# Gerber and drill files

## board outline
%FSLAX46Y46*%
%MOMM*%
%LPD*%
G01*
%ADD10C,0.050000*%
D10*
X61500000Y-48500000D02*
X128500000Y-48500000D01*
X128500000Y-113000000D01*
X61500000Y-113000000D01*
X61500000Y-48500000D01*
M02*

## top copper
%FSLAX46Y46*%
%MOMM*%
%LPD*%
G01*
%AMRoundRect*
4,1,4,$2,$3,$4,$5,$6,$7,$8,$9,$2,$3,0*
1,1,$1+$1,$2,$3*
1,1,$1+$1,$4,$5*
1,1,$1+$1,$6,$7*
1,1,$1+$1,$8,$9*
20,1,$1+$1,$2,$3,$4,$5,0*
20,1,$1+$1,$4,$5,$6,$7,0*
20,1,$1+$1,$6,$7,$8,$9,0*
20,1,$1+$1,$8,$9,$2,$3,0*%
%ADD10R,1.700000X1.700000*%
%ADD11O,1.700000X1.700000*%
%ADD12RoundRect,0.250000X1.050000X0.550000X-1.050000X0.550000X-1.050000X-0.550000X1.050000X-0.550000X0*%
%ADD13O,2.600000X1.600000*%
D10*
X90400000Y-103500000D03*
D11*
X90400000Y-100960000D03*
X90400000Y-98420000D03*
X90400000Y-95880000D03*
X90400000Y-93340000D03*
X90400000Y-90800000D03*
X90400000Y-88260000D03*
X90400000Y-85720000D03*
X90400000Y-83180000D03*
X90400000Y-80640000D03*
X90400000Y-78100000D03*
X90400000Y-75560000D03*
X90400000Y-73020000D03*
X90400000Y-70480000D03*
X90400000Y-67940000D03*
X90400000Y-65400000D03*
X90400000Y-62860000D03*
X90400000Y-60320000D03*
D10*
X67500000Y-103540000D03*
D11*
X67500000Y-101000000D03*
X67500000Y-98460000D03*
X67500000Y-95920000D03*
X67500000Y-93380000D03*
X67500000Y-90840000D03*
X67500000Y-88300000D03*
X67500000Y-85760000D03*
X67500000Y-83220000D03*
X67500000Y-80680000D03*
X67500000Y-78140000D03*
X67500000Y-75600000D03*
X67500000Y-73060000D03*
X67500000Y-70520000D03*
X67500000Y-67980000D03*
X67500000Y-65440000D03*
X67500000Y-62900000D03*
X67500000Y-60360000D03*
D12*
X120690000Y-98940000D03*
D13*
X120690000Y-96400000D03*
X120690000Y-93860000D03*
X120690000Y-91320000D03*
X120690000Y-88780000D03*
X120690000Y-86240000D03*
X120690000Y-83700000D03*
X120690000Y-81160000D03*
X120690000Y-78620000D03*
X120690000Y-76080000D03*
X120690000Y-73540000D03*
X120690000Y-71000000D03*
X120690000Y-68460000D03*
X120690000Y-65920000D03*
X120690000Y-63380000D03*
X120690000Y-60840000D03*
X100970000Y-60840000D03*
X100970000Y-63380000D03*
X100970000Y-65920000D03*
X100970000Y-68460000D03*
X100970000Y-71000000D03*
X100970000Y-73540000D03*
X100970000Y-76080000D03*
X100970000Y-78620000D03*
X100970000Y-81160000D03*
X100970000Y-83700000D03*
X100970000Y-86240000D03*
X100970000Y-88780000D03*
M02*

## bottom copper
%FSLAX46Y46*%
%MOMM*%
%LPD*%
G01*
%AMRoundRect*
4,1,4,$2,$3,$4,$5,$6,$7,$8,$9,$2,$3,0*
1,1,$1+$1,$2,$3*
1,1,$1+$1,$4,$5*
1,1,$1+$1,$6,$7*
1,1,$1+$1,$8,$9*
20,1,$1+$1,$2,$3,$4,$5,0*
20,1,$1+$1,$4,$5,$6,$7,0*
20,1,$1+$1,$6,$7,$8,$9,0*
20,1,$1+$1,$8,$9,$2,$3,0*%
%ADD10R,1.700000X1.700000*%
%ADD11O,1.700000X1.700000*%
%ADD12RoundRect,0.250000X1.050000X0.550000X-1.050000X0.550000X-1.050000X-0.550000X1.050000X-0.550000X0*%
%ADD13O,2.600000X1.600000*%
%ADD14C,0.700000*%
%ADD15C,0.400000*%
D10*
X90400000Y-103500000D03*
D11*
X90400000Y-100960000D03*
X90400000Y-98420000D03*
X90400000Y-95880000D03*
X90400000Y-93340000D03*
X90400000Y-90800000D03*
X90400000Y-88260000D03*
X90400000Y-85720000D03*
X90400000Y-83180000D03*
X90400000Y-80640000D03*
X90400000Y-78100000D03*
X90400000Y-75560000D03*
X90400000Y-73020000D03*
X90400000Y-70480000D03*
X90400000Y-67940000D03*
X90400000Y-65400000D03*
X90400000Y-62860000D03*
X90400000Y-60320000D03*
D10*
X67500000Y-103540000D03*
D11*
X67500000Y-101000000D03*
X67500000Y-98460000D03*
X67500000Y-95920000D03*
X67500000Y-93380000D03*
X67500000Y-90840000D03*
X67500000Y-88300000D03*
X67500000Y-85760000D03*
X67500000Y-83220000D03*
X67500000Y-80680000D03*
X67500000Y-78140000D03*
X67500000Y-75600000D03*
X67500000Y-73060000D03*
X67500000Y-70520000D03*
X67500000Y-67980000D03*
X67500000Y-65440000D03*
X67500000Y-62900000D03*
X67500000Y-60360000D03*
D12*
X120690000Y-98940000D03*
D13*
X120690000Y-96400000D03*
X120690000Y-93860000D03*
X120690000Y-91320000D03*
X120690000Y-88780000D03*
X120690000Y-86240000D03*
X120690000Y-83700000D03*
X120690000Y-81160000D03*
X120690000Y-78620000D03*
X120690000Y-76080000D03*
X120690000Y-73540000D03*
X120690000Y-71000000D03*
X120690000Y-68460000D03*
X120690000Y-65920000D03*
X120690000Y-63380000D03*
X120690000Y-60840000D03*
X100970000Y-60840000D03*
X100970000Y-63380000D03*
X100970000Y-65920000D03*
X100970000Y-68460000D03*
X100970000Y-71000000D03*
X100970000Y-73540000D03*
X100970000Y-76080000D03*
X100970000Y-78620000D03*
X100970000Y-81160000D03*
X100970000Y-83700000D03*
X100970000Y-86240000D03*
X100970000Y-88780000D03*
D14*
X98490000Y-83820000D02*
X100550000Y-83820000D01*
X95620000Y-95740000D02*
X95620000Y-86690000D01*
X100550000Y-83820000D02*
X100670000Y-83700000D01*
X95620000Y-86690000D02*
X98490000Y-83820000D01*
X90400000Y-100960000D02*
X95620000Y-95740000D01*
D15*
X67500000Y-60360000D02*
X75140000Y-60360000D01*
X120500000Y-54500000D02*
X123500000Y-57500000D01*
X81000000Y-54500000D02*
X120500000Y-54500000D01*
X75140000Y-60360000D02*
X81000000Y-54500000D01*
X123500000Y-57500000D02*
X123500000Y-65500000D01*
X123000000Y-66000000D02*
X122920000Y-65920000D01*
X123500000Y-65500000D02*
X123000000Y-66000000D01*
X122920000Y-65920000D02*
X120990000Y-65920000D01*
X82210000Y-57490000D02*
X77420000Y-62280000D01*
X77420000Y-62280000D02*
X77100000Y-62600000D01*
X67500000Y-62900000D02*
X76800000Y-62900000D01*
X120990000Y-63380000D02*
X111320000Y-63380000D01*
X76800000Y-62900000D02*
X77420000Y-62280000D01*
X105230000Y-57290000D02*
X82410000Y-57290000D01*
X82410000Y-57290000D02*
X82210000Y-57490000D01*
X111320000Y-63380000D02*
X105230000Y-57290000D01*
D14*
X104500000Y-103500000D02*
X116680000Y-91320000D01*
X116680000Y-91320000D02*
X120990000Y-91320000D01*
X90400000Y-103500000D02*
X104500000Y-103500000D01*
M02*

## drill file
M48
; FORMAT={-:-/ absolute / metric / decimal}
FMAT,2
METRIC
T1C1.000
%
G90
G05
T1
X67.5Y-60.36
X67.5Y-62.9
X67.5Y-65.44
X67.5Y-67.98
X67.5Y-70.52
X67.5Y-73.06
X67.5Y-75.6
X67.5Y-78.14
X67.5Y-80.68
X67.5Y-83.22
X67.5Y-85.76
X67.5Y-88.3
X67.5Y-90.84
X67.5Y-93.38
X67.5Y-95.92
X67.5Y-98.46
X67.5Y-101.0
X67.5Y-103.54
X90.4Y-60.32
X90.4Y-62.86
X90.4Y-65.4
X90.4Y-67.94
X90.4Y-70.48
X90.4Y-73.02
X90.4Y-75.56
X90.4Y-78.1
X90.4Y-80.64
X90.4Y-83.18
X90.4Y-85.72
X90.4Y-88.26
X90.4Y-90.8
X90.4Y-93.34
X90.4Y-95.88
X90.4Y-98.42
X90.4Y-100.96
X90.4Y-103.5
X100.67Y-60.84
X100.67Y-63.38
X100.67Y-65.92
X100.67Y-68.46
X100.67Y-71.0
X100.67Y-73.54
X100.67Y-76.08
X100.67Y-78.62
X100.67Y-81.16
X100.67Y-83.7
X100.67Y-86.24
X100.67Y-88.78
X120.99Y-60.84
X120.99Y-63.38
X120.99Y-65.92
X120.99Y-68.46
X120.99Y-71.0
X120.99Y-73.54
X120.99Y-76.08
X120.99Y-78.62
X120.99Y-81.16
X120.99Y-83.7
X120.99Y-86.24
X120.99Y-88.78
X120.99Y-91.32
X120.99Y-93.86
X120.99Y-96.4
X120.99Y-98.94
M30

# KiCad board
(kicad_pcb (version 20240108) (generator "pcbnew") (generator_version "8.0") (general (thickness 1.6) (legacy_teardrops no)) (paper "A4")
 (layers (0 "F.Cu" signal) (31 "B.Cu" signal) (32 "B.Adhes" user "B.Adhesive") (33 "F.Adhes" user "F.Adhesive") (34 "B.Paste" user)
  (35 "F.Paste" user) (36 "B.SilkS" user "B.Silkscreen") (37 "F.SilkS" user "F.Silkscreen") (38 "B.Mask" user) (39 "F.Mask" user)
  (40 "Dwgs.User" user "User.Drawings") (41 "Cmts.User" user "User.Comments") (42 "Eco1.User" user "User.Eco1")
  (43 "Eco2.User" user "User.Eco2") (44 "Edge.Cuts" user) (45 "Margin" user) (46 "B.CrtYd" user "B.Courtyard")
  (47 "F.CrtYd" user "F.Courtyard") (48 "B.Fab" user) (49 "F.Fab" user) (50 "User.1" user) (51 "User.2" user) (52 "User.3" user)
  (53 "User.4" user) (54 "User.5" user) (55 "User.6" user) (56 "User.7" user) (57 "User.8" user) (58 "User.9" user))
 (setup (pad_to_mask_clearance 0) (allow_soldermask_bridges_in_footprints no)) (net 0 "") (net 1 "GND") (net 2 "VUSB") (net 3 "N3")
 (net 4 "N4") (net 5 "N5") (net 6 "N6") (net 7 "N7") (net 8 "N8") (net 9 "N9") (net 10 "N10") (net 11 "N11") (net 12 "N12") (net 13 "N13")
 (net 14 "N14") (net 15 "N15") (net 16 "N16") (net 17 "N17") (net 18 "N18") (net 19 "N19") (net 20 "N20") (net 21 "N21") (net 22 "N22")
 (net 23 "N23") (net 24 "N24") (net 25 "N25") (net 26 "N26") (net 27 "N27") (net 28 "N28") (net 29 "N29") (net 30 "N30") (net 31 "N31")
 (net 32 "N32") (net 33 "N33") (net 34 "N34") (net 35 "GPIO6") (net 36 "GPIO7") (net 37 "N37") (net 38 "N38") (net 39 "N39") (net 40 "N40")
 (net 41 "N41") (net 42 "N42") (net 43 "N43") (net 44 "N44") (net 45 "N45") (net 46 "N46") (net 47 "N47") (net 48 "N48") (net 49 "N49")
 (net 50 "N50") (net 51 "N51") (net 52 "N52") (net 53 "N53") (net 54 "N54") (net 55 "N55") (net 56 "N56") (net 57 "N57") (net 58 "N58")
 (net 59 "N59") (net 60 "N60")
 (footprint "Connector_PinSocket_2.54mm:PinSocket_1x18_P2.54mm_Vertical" (layer "F.Cu") (at 90.4 103.5 180)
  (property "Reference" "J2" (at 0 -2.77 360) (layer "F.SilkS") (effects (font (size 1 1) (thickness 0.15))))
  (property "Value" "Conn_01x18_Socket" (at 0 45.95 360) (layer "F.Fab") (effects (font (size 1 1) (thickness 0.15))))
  (pad "1" thru_hole rect (at 0 0 180) (size 1.7 1.7) (drill 1) (layers "*.Cu" "*.Mask") (remove_unused_layers no) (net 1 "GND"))
  (pad "2" thru_hole oval (at 0 2.54 180) (size 1.7 1.7) (drill 1) (layers "*.Cu" "*.Mask") (remove_unused_layers no) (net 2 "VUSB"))
  (pad "3" thru_hole oval (at 0 5.08 180) (size 1.7 1.7) (drill 1) (layers "*.Cu" "*.Mask") (remove_unused_layers no) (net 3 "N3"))
  (pad "4" thru_hole oval (at 0 7.62 180) (size 1.7 1.7) (drill 1) (layers "*.Cu" "*.Mask") (remove_unused_layers no) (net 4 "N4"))
  (pad "5" thru_hole oval (at 0 10.16 180) (size 1.7 1.7) (drill 1) (layers "*.Cu" "*.Mask") (remove_unused_layers no) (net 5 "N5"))
  (pad "6" thru_hole oval (at 0 12.7 180) (size 1.7 1.7) (drill 1) (layers "*.Cu" "*.Mask") (remove_unused_layers no) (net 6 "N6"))
  (pad "7" thru_hole oval (at 0 15.24 180) (size 1.7 1.7) (drill 1) (layers "*.Cu" "*.Mask") (remove_unused_layers no) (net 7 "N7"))
  (pad "8" thru_hole oval (at 0 17.78 180) (size 1.7 1.7) (drill 1) (layers "*.Cu" "*.Mask") (remove_unused_layers no) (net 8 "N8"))
  (pad "9" thru_hole oval (at 0 20.32 180) (size 1.7 1.7) (drill 1) (layers "*.Cu" "*.Mask") (remove_unused_layers no) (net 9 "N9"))
  (pad "10" thru_hole oval (at 0 22.86 180) (size 1.7 1.7) (drill 1) (layers "*.Cu" "*.Mask") (remove_unused_layers no) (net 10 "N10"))
  (pad "11" thru_hole oval (at 0 25.4 180) (size 1.7 1.7) (drill 1) (layers "*.Cu" "*.Mask") (remove_unused_layers no) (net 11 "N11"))
  (pad "12" thru_hole oval (at 0 27.94 180) (size 1.7 1.7) (drill 1) (layers "*.Cu" "*.Mask") (remove_unused_layers no) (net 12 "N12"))
  (pad "13" thru_hole oval (at 0 30.48 180) (size 1.7 1.7) (drill 1) (layers "*.Cu" "*.Mask") (remove_unused_layers no) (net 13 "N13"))
  (pad "14" thru_hole oval (at 0 33.02 180) (size 1.7 1.7) (drill 1) (layers "*.Cu" "*.Mask") (remove_unused_layers no) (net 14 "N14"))
  (pad "15" thru_hole oval (at 0 35.56 180) (size 1.7 1.7) (drill 1) (layers "*.Cu" "*.Mask") (remove_unused_layers no) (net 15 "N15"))
  (pad "16" thru_hole oval (at 0 38.1 180) (size 1.7 1.7) (drill 1) (layers "*.Cu" "*.Mask") (remove_unused_layers no) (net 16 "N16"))
  (pad "17" thru_hole oval (at 0 40.64 180) (size 1.7 1.7) (drill 1) (layers "*.Cu" "*.Mask") (remove_unused_layers no) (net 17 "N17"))
  (pad "18" thru_hole oval (at 0 43.18 180) (size 1.7 1.7) (drill 1) (layers "*.Cu" "*.Mask") (remove_unused_layers no) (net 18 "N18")))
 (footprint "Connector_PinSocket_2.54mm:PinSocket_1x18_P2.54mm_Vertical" (layer "F.Cu") (at 67.5 103.54 180)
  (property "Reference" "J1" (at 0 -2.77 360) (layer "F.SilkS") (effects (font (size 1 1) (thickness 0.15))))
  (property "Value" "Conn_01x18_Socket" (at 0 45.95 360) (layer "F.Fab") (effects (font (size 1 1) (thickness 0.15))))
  (pad "1" thru_hole rect (at 0 0 180) (size 1.7 1.7) (drill 1) (layers "*.Cu" "*.Mask") (remove_unused_layers no) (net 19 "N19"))
  (pad "2" thru_hole oval (at 0 2.54 180) (size 1.7 1.7) (drill 1) (layers "*.Cu" "*.Mask") (remove_unused_layers no) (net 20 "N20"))
  (pad "3" thru_hole oval (at 0 5.08 180) (size 1.7 1.7) (drill 1) (layers "*.Cu" "*.Mask") (remove_unused_layers no) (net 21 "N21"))
  (pad "4" thru_hole oval (at 0 7.62 180) (size 1.7 1.7) (drill 1) (layers "*.Cu" "*.Mask") (remove_unused_layers no) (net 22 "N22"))
  (pad "5" thru_hole oval (at 0 10.16 180) (size 1.7 1.7) (drill 1) (layers "*.Cu" "*.Mask") (remove_unused_layers no) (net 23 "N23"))
  (pad "6" thru_hole oval (at 0 12.7 180) (size 1.7 1.7) (drill 1) (layers "*.Cu" "*.Mask") (remove_unused_layers no) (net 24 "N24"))
  (pad "7" thru_hole oval (at 0 15.24 180) (size 1.7 1.7) (drill 1) (layers "*.Cu" "*.Mask") (remove_unused_layers no) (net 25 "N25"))
  (pad "8" thru_hole oval (at 0 17.78 180) (size 1.7 1.7) (drill 1) (layers "*.Cu" "*.Mask") (remove_unused_layers no) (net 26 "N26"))
  (pad "9" thru_hole oval (at 0 20.32 180) (size 1.7 1.7) (drill 1) (layers "*.Cu" "*.Mask") (remove_unused_layers no) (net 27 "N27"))
  (pad "10" thru_hole oval (at 0 22.86 180) (size 1.7 1.7) (drill 1) (layers "*.Cu" "*.Mask") (remove_unused_layers no) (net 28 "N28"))
  (pad "11" thru_hole oval (at 0 25.4 180) (size 1.7 1.7) (drill 1) (layers "*.Cu" "*.Mask") (remove_unused_layers no) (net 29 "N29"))
  (pad "12" thru_hole oval (at 0 27.94 180) (size 1.7 1.7) (drill 1) (layers "*.Cu" "*.Mask") (remove_unused_layers no) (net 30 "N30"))
  (pad "13" thru_hole oval (at 0 30.48 180) (size 1.7 1.7) (drill 1) (layers "*.Cu" "*.Mask") (remove_unused_layers no) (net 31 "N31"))
  (pad "14" thru_hole oval (at 0 33.02 180) (size 1.7 1.7) (drill 1) (layers "*.Cu" "*.Mask") (remove_unused_layers no) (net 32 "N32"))
  (pad "15" thru_hole oval (at 0 35.56 180) (size 1.7 1.7) (drill 1) (layers "*.Cu" "*.Mask") (remove_unused_layers no) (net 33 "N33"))
  (pad "16" thru_hole oval (at 0 38.1 180) (size 1.7 1.7) (drill 1) (layers "*.Cu" "*.Mask") (remove_unused_layers no) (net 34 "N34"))
  (pad "17" thru_hole oval (at 0 40.64 180) (size 1.7 1.7) (drill 1) (layers "*.Cu" "*.Mask") (remove_unused_layers no) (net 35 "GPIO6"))
  (pad "18" thru_hole oval (at 0 43.18 180) (size 1.7 1.7) (drill 1) (layers "*.Cu" "*.Mask") (remove_unused_layers no) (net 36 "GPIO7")))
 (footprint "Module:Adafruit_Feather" (layer "F.Cu") (at 120.99 98.94 180)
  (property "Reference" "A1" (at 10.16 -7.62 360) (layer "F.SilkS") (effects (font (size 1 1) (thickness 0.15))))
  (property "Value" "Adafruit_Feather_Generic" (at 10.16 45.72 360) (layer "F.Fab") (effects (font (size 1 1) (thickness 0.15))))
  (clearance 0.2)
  (pad "1" thru_hole roundrect (at 0 0 180) (size 2.6 1.6) (drill 1 (offset 0.3 0)) (layers "*.Cu" "*.Mask") (remove_unused_layers no)
   (roundrect_rratio 0.15625) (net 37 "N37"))
  (pad "2" thru_hole oval (at 0 2.54 180) (size 2.6 1.6) (drill 1 (offset 0.3 0)) (layers "*.Cu" "*.Mask") (remove_unused_layers no)
   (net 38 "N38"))
  (pad "3" thru_hole oval (at 0 5.08 180) (size 2.6 1.6) (drill 1 (offset 0.3 0)) (layers "*.Cu" "*.Mask") (remove_unused_layers no)
   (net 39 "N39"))
  (pad "4" thru_hole oval (at 0 7.62 180) (size 2.6 1.6) (drill 1 (offset 0.3 0)) (layers "*.Cu" "*.Mask") (remove_unused_layers no)
   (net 1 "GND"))
  (pad "5" thru_hole oval (at 0 10.16 180) (size 2.6 1.6) (drill 1 (offset 0.3 0)) (layers "*.Cu" "*.Mask") (remove_unused_layers no)
   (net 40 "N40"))
  (pad "6" thru_hole oval (at 0 12.7 180) (size 2.6 1.6) (drill 1 (offset 0.3 0)) (layers "*.Cu" "*.Mask") (remove_unused_layers no)
   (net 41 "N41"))
  (pad "7" thru_hole oval (at 0 15.24 180) (size 2.6 1.6) (drill 1 (offset 0.3 0)) (layers "*.Cu" "*.Mask") (remove_unused_layers no)
   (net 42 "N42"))
  (pad "8" thru_hole oval (at 0 17.78 180) (size 2.6 1.6) (drill 1 (offset 0.3 0)) (layers "*.Cu" "*.Mask") (remove_unused_layers no)
   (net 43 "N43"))
  (pad "9" thru_hole oval (at 0 20.32 180) (size 2.6 1.6) (drill 1 (offset 0.3 0)) (layers "*.Cu" "*.Mask") (remove_unused_layers no)
   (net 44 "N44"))
  (pad "10" thru_hole oval (at 0 22.86 180) (size 2.6 1.6) (drill 1 (offset 0.3 0)) (layers "*.Cu" "*.Mask") (remove_unused_layers no)
   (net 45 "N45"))
  (pad "11" thru_hole oval (at 0 25.4 180) (size 2.6 1.6) (drill 1 (offset 0.3 0)) (layers "*.Cu" "*.Mask") (remove_unused_layers no)
   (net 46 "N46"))
  (pad "12" thru_hole oval (at 0 27.94 180) (size 2.6 1.6) (drill 1 (offset 0.3 0)) (layers "*.Cu" "*.Mask") (remove_unused_layers no)
   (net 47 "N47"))
  (pad "13" thru_hole oval (at 0 30.48 180) (size 2.6 1.6) (drill 1 (offset 0.3 0)) (layers "*.Cu" "*.Mask") (remove_unused_layers no)
   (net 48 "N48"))
  (pad "14" thru_hole oval (at 0 33.02 180) (size 2.6 1.6) (drill 1 (offset 0.3 0)) (layers "*.Cu" "*.Mask") (remove_unused_layers no)
   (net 36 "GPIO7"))
  (pad "15" thru_hole oval (at 0 35.56 180) (size 2.6 1.6) (drill 1 (offset 0.3 0)) (layers "*.Cu" "*.Mask") (remove_unused_layers no)
   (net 35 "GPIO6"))
  (pad "16" thru_hole oval (at 0 38.1 180) (size 2.6 1.6) (drill 1 (offset 0.3 0)) (layers "*.Cu" "*.Mask") (remove_unused_layers no)
   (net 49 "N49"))
  (pad "17" thru_hole oval (at 20.32 38.1) (size 2.6 1.6) (drill 1 (offset 0.3 0)) (layers "*.Cu" "*.Mask") (remove_unused_layers no)
   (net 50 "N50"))
  (pad "18" thru_hole oval (at 20.32 35.56) (size 2.6 1.6) (drill 1 (offset 0.3 0)) (layers "*.Cu" "*.Mask") (remove_unused_layers no)
   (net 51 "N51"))
  (pad "19" thru_hole oval (at 20.32 33.02) (size 2.6 1.6) (drill 1 (offset 0.3 0)) (layers "*.Cu" "*.Mask") (remove_unused_layers no)
   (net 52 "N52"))
  (pad "20" thru_hole oval (at 20.32 30.48) (size 2.6 1.6) (drill 1 (offset 0.3 0)) (layers "*.Cu" "*.Mask") (remove_unused_layers no)
   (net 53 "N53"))
  (pad "21" thru_hole oval (at 20.32 27.94) (size 2.6 1.6) (drill 1 (offset 0.3 0)) (layers "*.Cu" "*.Mask") (remove_unused_layers no)
   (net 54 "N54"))
  (pad "22" thru_hole oval (at 20.32 25.4) (size 2.6 1.6) (drill 1 (offset 0.3 0)) (layers "*.Cu" "*.Mask") (remove_unused_layers no)
   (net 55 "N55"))
  (pad "23" thru_hole oval (at 20.32 22.86) (size 2.6 1.6) (drill 1 (offset 0.3 0)) (layers "*.Cu" "*.Mask") (remove_unused_layers no)
   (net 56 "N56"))
  (pad "24" thru_hole oval (at 20.32 20.32) (size 2.6 1.6) (drill 1 (offset 0.3 0)) (layers "*.Cu" "*.Mask") (remove_unused_layers no)
   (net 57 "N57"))
  (pad "25" thru_hole oval (at 20.32 17.78) (size 2.6 1.6) (drill 1 (offset 0.3 0)) (layers "*.Cu" "*.Mask") (remove_unused_layers no)
   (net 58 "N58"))
  (pad "26" thru_hole oval (at 20.32 15.24) (size 2.6 1.6) (drill 1 (offset 0.3 0)) (layers "*.Cu" "*.Mask") (remove_unused_layers no)
   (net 2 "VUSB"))
  (pad "27" thru_hole oval (at 20.32 12.7) (size 2.6 1.6) (drill 1 (offset 0.3 0)) (layers "*.Cu" "*.Mask") (remove_unused_layers no)
   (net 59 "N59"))
  (pad "28" thru_hole oval (at 20.32 10.16) (size 2.6 1.6) (drill 1 (offset 0.3 0)) (layers "*.Cu" "*.Mask") (remove_unused_layers no)
   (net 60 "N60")))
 (gr_rect (start 61.5 48.5) (end 128.5 113) (stroke (width 0.05) (type default)) (fill none) (layer "Edge.Cuts"))
 (segment (start 98.49 83.82) (end 100.55 83.82) (width 0.7) (layer "B.Cu") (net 2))
 (segment (start 95.62 95.74) (end 95.62 86.69) (width 0.7) (layer "B.Cu") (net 2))
 (segment (start 100.55 83.82) (end 100.67 83.7) (width 0.7) (layer "B.Cu") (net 2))
 (segment (start 95.62 86.69) (end 98.49 83.82) (width 0.7) (layer "B.Cu") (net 2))
 (segment (start 90.4 100.96) (end 95.62 95.74) (width 0.7) (layer "B.Cu") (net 2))
 (segment (start 67.5 60.36) (end 75.14 60.36) (width 0.4) (layer "B.Cu") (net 36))
 (segment (start 120.5 54.5) (end 123.5 57.5) (width 0.4) (layer "B.Cu") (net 36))
 (segment (start 81 54.5) (end 120.5 54.5) (width 0.4) (layer "B.Cu") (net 36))
 (segment (start 75.14 60.36) (end 81 54.5) (width 0.4) (layer "B.Cu") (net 36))
 (segment (start 123.5 57.5) (end 123.5 65.5) (width 0.4) (layer "B.Cu") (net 36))
 (segment (start 123 66) (end 122.92 65.92) (width 0.4) (layer "B.Cu") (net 36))
 (segment (start 123.5 65.5) (end 123 66) (width 0.4) (layer "B.Cu") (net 36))
 (segment (start 122.92 65.92) (end 120.99 65.92) (width 0.4) (layer "B.Cu") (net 36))
 (segment (start 82.21 57.49) (end 77.42 62.28) (width 0.4) (layer "B.Cu") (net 35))
 (segment (start 77.42 62.28) (end 77.1 62.6) (width 0.4) (layer "B.Cu") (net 35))
 (segment (start 67.5 62.9) (end 76.8 62.9) (width 0.4) (layer "B.Cu") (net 35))
 (segment (start 120.99 63.38) (end 111.32 63.38) (width 0.4) (layer "B.Cu") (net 35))
 (segment (start 76.8 62.9) (end 77.42 62.28) (width 0.4) (layer "B.Cu") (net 35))
 (segment (start 105.23 57.29) (end 82.41 57.29) (width 0.4) (layer "B.Cu") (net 35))
 (segment (start 82.41 57.29) (end 82.21 57.49) (width 0.4) (layer "B.Cu") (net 35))
 (segment (start 111.32 63.38) (end 105.23 57.29) (width 0.4) (layer "B.Cu") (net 35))
 (segment (start 104.5 103.5) (end 116.68 91.32) (width 0.7) (layer "B.Cu") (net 1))
 (segment (start 116.68 91.32) (end 120.99 91.32) (width 0.7) (layer "B.Cu") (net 1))
 (segment (start 90.4 103.5) (end 104.5 103.5) (width 0.7) (layer "B.Cu") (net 1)))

